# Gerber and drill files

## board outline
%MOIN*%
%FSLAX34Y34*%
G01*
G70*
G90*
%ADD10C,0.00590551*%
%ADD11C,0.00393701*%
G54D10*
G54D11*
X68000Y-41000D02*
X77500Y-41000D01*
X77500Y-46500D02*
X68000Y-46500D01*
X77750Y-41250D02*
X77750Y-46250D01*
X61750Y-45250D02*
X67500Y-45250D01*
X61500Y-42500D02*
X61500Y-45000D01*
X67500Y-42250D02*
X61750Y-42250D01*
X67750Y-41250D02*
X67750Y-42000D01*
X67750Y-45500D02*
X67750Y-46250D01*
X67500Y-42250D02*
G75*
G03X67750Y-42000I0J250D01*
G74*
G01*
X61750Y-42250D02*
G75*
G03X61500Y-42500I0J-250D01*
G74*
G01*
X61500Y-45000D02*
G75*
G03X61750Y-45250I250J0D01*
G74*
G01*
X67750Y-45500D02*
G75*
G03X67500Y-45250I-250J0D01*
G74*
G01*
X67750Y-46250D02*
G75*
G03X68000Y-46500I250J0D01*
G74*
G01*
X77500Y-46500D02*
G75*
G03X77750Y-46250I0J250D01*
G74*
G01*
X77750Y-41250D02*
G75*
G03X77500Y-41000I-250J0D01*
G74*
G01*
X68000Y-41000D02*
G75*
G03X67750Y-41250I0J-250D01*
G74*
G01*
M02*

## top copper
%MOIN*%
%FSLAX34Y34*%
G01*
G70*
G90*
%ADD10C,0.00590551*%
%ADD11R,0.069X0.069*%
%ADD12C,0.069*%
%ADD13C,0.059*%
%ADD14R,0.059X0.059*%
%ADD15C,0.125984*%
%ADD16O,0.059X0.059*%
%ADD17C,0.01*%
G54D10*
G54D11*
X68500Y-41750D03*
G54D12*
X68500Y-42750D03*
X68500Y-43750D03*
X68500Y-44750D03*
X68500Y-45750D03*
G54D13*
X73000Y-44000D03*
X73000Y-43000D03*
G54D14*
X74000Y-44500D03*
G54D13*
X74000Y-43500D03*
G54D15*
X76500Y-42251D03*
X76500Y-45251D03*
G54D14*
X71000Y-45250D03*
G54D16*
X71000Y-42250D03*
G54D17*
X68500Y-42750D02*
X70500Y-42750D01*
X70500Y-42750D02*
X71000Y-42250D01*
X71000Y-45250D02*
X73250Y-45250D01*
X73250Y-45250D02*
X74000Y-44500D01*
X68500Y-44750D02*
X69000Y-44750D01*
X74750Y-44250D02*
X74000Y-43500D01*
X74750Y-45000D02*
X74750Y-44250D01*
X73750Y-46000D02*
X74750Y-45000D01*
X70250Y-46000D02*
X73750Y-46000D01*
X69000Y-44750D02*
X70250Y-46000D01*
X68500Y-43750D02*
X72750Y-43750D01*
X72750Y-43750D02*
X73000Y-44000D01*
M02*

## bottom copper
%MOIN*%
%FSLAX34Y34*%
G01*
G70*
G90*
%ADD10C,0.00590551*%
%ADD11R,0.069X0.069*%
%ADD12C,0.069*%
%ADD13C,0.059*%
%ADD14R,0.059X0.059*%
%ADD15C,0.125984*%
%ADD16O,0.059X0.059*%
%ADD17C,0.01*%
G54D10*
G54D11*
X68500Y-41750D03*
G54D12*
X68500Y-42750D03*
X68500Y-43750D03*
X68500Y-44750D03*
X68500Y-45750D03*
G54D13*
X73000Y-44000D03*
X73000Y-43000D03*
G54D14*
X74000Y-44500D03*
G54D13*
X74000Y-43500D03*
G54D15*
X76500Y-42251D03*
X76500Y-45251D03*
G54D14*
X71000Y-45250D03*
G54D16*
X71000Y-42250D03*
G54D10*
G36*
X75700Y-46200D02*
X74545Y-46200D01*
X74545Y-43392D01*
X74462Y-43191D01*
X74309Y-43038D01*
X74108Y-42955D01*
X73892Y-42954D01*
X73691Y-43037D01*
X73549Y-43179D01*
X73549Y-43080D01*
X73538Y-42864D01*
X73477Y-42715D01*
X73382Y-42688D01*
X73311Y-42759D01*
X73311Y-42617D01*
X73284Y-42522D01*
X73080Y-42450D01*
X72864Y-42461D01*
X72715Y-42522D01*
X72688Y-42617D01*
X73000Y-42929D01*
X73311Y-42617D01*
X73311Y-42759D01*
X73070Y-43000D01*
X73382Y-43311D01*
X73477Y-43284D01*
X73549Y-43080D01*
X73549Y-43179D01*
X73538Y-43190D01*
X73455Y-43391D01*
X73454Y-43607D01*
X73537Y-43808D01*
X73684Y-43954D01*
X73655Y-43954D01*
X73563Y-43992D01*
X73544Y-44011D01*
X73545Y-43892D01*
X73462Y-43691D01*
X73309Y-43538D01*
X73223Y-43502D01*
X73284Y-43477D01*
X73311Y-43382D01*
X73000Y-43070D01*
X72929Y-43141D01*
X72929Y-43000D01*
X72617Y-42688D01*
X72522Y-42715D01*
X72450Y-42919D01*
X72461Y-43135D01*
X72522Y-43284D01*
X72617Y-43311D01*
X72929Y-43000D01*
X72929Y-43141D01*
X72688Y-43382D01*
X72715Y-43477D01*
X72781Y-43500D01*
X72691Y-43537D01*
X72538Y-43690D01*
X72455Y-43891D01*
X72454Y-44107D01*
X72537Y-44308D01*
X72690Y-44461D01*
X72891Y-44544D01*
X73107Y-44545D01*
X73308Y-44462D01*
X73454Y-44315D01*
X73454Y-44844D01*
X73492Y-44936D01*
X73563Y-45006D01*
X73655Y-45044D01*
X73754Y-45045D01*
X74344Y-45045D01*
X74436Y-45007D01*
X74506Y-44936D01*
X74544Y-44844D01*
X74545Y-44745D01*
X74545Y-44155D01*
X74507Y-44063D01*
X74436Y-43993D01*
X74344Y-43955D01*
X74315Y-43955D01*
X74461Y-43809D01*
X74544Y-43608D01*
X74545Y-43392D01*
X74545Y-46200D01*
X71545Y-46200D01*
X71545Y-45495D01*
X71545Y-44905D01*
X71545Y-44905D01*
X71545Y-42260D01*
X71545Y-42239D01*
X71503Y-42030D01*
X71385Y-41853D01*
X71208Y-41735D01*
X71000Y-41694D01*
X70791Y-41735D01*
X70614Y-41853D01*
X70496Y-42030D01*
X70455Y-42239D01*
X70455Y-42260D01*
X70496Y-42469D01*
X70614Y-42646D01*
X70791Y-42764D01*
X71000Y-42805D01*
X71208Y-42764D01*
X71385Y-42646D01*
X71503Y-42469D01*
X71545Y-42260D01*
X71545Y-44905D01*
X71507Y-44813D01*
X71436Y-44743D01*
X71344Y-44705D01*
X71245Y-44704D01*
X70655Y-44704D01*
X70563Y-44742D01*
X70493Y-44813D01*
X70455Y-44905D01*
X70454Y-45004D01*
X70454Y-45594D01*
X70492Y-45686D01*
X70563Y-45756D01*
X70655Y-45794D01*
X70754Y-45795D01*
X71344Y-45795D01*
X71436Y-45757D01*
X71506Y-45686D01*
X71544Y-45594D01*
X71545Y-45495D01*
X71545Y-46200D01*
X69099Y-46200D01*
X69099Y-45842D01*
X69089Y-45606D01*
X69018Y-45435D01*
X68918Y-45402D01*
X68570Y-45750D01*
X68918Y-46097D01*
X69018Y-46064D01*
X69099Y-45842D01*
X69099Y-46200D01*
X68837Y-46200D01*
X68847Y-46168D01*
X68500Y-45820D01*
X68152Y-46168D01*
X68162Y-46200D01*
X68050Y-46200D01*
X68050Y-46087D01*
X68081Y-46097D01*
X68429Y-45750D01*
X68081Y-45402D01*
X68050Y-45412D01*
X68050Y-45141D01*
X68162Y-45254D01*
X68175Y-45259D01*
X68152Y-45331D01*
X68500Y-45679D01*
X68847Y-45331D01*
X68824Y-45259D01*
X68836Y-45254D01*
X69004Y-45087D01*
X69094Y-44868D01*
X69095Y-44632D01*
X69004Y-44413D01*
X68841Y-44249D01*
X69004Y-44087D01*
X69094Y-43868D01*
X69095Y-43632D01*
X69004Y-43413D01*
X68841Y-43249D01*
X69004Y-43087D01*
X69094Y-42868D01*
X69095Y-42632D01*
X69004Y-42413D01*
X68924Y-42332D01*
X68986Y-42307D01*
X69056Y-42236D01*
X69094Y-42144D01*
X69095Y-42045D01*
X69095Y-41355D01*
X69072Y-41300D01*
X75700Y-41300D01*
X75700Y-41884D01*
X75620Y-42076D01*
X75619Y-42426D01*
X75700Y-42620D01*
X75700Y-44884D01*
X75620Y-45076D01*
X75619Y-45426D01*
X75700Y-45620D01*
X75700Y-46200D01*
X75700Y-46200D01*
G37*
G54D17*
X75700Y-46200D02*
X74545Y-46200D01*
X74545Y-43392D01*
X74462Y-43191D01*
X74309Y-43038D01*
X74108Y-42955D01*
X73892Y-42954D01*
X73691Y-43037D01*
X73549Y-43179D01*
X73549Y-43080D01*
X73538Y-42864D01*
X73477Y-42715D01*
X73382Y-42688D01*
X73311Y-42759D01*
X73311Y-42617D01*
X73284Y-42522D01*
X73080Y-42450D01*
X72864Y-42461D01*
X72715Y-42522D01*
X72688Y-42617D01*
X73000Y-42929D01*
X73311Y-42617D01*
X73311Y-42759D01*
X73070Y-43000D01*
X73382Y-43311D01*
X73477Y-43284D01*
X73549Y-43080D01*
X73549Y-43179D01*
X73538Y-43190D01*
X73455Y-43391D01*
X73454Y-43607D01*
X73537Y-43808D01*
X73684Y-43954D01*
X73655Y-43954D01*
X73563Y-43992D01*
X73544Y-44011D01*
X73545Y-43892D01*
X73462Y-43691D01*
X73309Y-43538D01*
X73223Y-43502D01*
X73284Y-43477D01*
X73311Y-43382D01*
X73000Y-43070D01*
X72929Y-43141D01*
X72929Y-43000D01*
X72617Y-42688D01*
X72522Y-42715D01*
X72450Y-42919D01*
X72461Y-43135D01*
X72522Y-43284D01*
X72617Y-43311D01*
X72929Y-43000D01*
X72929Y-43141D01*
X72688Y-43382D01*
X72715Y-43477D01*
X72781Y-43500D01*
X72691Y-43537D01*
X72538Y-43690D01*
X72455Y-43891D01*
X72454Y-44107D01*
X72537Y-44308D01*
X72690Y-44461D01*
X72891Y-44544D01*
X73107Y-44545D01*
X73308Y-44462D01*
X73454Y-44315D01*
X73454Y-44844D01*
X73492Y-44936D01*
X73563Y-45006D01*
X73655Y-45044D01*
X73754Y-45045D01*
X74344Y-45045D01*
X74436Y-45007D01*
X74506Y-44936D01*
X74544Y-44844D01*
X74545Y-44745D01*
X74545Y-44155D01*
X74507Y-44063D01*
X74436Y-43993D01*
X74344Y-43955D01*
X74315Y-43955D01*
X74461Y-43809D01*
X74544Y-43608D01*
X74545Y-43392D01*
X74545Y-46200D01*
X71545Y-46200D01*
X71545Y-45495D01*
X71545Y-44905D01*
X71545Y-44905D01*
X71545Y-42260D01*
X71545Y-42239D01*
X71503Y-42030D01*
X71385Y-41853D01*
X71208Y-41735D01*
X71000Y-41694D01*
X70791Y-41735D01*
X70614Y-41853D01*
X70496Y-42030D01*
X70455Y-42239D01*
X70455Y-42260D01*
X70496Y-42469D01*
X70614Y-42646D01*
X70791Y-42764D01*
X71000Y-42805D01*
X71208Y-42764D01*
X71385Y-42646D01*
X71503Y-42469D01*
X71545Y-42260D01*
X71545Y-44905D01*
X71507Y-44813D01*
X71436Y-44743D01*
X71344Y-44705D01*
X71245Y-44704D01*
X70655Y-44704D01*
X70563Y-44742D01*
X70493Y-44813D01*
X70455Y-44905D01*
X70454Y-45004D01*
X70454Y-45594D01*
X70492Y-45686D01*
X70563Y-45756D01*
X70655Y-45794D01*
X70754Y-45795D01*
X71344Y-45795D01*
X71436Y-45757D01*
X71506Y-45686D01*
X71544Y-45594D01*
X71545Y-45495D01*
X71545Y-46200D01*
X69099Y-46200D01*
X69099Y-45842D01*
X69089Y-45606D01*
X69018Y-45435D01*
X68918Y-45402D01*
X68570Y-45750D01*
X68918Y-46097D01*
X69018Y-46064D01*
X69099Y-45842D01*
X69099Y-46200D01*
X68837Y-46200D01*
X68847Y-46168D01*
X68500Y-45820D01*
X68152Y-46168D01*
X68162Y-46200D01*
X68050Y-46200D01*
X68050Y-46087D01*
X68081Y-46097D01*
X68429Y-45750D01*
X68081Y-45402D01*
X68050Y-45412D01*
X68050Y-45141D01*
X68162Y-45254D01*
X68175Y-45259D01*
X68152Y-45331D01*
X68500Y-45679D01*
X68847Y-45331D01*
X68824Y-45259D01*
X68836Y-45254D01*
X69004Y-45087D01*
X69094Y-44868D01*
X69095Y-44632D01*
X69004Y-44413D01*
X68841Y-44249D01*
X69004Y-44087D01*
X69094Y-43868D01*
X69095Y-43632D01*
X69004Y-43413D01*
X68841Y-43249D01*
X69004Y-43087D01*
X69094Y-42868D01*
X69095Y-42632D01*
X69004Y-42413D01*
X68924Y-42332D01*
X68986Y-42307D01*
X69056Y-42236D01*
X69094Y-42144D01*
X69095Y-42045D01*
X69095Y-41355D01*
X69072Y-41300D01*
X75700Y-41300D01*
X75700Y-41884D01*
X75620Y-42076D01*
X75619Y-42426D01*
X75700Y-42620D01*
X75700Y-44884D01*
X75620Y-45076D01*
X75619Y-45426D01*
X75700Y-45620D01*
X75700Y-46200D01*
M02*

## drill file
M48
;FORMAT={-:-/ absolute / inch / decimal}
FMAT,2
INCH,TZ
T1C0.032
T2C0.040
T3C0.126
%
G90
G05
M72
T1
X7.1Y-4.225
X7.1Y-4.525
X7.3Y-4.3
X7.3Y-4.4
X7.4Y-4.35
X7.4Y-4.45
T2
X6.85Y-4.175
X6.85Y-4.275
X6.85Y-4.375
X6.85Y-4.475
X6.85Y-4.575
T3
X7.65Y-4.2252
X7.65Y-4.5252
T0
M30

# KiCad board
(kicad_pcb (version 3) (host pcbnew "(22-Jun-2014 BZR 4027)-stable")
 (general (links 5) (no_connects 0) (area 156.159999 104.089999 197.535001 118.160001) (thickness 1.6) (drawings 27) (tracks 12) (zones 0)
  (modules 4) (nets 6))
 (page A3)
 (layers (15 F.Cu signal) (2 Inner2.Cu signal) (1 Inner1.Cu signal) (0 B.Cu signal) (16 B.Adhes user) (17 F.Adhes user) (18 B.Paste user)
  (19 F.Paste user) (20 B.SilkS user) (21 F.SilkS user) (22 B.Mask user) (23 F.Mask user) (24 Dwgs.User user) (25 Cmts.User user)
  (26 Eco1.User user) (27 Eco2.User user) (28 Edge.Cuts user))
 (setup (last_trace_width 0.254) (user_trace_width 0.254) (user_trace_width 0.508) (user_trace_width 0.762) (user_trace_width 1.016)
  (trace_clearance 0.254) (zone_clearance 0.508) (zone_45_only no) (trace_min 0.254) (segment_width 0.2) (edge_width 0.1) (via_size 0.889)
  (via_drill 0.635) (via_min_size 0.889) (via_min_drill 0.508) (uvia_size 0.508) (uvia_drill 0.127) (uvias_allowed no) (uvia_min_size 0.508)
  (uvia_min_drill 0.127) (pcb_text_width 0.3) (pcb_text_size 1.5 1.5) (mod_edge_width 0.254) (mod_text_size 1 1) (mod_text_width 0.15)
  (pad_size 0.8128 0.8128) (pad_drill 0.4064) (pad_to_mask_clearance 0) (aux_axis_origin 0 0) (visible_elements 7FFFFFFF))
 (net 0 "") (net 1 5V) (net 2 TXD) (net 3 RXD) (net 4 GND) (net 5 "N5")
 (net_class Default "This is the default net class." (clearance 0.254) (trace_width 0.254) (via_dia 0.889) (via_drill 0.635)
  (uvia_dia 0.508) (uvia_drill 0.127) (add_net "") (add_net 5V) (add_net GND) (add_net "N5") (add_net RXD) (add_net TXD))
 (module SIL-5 (layer F.Cu) (at 173.99 108.585 270)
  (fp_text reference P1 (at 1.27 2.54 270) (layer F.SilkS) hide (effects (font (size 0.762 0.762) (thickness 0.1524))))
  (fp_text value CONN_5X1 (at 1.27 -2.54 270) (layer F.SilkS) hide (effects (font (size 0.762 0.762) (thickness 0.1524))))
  (pad 1 thru_hole rect (at -2.54 0 270) (size 1.7526 1.7526) (drill 1.016) (layers *.Cu *.Mask F.SilkS))
  (pad 2 thru_hole circle (at 0 0 270) (size 1.7526 1.7526) (drill 1.016) (layers *.Cu *.Mask F.SilkS) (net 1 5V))
  (pad 3 thru_hole circle (at 2.54 0 270) (size 1.7526 1.7526) (drill 1.016) (layers *.Cu *.Mask F.SilkS) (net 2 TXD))
  (pad 4 thru_hole circle (at 5.08 0 270) (size 1.7526 1.7526) (drill 1.016) (layers *.Cu *.Mask F.SilkS) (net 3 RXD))
  (pad 5 thru_hole circle (at 7.62 0 270) (size 1.7526 1.7526) (drill 1.016) (layers *.Cu *.Mask F.SilkS) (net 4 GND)))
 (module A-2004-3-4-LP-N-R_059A (layer F.Cu) (at 187.96 113.03 90)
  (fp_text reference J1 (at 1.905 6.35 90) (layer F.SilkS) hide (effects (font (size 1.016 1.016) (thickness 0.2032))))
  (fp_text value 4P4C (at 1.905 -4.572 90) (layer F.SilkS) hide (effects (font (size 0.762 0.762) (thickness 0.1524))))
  (pad 2 thru_hole circle (at 1.27 -2.54 90) (size 1.4986 1.4986) (drill 0.8128) (layers *.Cu *.Mask F.SilkS) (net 2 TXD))
  (pad 4 thru_hole circle (at 3.81 -2.54 90) (size 1.4986 1.4986) (drill 0.8128) (layers *.Cu *.Mask F.SilkS) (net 4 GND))
  (pad 1 thru_hole rect (at 0 0 90) (size 1.4986 1.4986) (drill 0.8128) (layers *.Cu *.Mask F.SilkS) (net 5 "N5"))
  (pad 3 thru_hole circle (at 2.54 0 90) (size 1.4986 1.4986) (drill 0.8128) (layers *.Cu *.Mask F.SilkS) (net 3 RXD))
  (pad "" thru_hole circle (at 5.71 6.35 90) (size 3.2 3.2) (drill 3.2) (layers *.Cu *.Mask F.SilkS))
  (pad "" thru_hole circle (at -1.91 6.35 90) (size 3.2 3.2) (drill 3.2) (layers *.Cu *.Mask F.SilkS)))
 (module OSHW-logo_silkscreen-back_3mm (layer F.Cu) (at 169.545 111.125)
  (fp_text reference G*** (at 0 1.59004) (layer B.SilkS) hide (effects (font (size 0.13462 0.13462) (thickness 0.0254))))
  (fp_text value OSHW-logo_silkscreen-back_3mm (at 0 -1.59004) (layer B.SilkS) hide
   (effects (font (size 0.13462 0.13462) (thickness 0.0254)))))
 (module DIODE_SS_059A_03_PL (layer F.Cu) (at 180.34 111.125 270)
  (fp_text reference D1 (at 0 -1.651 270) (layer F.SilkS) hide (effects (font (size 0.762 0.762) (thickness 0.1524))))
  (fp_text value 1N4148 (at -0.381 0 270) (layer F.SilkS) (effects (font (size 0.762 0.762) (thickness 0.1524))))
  (pad 2 thru_hole rect (at 3.81 0 270) (size 1.4986 1.4986) (drill 0.8128) (layers *.Cu *.Mask F.SilkS) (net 5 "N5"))
  (pad 1 thru_hole oval (at -3.81 0 270) (size 1.4986 1.4986) (drill 0.8128) (layers *.Cu *.Mask F.SilkS) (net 1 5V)))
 (gr_line (start 172.72 104.14) (end 196.85 104.14) (angle 90) (layer Edge.Cuts) (width 0.1))
 (gr_line (start 196.85 118.11) (end 172.72 118.11) (angle 90) (layer Edge.Cuts) (width 0.1))
 (gr_line (start 197.485 104.775) (end 197.485 117.475) (angle 90) (layer Edge.Cuts) (width 0.1))
 (gr_line (start 156.845 114.935) (end 171.45 114.935) (angle 90) (layer Edge.Cuts) (width 0.1))
 (gr_line (start 156.21 107.95) (end 156.21 114.3) (angle 90) (layer Edge.Cuts) (width 0.1))
 (gr_line (start 171.45 107.315) (end 156.845 107.315) (angle 90) (layer Edge.Cuts) (width 0.1))
 (gr_line (start 172.085 104.775) (end 172.085 106.68) (angle 90) (layer Edge.Cuts) (width 0.1))
 (gr_line (start 172.085 115.57) (end 172.085 117.475) (angle 90) (layer Edge.Cuts) (width 0.1))
 (gr_arc (start 171.45 106.68) (end 172.085 106.68) (angle 90) (layer Edge.Cuts) (width 0.1))
 (gr_arc (start 156.845 107.95) (end 156.21 107.95) (angle 90) (layer Edge.Cuts) (width 0.1))
 (gr_arc (start 156.845 114.3) (end 156.845 114.935) (angle 90) (layer Edge.Cuts) (width 0.1))
 (gr_arc (start 171.45 115.57) (end 171.45 114.935) (angle 90) (layer Edge.Cuts) (width 0.1))
 (gr_arc (start 172.72 117.475) (end 172.72 118.11) (angle 90) (layer Edge.Cuts) (width 0.1))
 (gr_arc (start 196.85 117.475) (end 197.485 117.475) (angle 90) (layer Edge.Cuts) (width 0.1))
 (gr_arc (start 196.85 104.775) (end 196.85 104.14) (angle 90) (layer Edge.Cuts) (width 0.1))
 (gr_arc (start 172.72 104.775) (end 172.085 104.775) (angle 90) (layer Edge.Cuts) (width 0.1))
 (segment (start 173.99 108.585) (end 179.07 108.585) (width 0.254) (layer F.Cu) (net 1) (status 400000))
 (segment (start 179.07 108.585) (end 180.34 107.315) (width 0.254) (layer F.Cu) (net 1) (status 800000))
 (segment (start 180.34 114.935) (end 186.055 114.935) (width 0.254) (layer F.Cu) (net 5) (status 400000))
 (segment (start 186.055 114.935) (end 187.96 113.03) (width 0.254) (layer F.Cu) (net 5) (status 800000))
 (segment (start 173.99 113.665) (end 175.26 113.665) (width 0.254) (layer F.Cu) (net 3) (status 400000))
 (segment (start 189.865 112.395) (end 187.96 110.49) (width 0.254) (layer F.Cu) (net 3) (status 800000))
 (segment (start 189.865 114.3) (end 189.865 112.395) (width 0.254) (layer F.Cu) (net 3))
 (segment (start 187.325 116.84) (end 189.865 114.3) (width 0.254) (layer F.Cu) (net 3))
 (segment (start 178.435 116.84) (end 187.325 116.84) (width 0.254) (layer F.Cu) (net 3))
 (segment (start 175.26 113.665) (end 178.435 116.84) (width 0.254) (layer F.Cu) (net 3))
 (segment (start 173.99 111.125) (end 184.785 111.125) (width 0.254) (layer F.Cu) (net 2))
 (segment (start 184.785 111.125) (end 185.42 111.76) (width 0.254) (layer F.Cu) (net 2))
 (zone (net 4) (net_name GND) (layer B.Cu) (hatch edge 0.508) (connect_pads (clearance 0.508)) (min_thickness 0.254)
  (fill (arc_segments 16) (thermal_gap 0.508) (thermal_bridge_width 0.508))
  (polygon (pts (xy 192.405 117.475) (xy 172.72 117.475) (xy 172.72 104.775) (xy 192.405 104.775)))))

